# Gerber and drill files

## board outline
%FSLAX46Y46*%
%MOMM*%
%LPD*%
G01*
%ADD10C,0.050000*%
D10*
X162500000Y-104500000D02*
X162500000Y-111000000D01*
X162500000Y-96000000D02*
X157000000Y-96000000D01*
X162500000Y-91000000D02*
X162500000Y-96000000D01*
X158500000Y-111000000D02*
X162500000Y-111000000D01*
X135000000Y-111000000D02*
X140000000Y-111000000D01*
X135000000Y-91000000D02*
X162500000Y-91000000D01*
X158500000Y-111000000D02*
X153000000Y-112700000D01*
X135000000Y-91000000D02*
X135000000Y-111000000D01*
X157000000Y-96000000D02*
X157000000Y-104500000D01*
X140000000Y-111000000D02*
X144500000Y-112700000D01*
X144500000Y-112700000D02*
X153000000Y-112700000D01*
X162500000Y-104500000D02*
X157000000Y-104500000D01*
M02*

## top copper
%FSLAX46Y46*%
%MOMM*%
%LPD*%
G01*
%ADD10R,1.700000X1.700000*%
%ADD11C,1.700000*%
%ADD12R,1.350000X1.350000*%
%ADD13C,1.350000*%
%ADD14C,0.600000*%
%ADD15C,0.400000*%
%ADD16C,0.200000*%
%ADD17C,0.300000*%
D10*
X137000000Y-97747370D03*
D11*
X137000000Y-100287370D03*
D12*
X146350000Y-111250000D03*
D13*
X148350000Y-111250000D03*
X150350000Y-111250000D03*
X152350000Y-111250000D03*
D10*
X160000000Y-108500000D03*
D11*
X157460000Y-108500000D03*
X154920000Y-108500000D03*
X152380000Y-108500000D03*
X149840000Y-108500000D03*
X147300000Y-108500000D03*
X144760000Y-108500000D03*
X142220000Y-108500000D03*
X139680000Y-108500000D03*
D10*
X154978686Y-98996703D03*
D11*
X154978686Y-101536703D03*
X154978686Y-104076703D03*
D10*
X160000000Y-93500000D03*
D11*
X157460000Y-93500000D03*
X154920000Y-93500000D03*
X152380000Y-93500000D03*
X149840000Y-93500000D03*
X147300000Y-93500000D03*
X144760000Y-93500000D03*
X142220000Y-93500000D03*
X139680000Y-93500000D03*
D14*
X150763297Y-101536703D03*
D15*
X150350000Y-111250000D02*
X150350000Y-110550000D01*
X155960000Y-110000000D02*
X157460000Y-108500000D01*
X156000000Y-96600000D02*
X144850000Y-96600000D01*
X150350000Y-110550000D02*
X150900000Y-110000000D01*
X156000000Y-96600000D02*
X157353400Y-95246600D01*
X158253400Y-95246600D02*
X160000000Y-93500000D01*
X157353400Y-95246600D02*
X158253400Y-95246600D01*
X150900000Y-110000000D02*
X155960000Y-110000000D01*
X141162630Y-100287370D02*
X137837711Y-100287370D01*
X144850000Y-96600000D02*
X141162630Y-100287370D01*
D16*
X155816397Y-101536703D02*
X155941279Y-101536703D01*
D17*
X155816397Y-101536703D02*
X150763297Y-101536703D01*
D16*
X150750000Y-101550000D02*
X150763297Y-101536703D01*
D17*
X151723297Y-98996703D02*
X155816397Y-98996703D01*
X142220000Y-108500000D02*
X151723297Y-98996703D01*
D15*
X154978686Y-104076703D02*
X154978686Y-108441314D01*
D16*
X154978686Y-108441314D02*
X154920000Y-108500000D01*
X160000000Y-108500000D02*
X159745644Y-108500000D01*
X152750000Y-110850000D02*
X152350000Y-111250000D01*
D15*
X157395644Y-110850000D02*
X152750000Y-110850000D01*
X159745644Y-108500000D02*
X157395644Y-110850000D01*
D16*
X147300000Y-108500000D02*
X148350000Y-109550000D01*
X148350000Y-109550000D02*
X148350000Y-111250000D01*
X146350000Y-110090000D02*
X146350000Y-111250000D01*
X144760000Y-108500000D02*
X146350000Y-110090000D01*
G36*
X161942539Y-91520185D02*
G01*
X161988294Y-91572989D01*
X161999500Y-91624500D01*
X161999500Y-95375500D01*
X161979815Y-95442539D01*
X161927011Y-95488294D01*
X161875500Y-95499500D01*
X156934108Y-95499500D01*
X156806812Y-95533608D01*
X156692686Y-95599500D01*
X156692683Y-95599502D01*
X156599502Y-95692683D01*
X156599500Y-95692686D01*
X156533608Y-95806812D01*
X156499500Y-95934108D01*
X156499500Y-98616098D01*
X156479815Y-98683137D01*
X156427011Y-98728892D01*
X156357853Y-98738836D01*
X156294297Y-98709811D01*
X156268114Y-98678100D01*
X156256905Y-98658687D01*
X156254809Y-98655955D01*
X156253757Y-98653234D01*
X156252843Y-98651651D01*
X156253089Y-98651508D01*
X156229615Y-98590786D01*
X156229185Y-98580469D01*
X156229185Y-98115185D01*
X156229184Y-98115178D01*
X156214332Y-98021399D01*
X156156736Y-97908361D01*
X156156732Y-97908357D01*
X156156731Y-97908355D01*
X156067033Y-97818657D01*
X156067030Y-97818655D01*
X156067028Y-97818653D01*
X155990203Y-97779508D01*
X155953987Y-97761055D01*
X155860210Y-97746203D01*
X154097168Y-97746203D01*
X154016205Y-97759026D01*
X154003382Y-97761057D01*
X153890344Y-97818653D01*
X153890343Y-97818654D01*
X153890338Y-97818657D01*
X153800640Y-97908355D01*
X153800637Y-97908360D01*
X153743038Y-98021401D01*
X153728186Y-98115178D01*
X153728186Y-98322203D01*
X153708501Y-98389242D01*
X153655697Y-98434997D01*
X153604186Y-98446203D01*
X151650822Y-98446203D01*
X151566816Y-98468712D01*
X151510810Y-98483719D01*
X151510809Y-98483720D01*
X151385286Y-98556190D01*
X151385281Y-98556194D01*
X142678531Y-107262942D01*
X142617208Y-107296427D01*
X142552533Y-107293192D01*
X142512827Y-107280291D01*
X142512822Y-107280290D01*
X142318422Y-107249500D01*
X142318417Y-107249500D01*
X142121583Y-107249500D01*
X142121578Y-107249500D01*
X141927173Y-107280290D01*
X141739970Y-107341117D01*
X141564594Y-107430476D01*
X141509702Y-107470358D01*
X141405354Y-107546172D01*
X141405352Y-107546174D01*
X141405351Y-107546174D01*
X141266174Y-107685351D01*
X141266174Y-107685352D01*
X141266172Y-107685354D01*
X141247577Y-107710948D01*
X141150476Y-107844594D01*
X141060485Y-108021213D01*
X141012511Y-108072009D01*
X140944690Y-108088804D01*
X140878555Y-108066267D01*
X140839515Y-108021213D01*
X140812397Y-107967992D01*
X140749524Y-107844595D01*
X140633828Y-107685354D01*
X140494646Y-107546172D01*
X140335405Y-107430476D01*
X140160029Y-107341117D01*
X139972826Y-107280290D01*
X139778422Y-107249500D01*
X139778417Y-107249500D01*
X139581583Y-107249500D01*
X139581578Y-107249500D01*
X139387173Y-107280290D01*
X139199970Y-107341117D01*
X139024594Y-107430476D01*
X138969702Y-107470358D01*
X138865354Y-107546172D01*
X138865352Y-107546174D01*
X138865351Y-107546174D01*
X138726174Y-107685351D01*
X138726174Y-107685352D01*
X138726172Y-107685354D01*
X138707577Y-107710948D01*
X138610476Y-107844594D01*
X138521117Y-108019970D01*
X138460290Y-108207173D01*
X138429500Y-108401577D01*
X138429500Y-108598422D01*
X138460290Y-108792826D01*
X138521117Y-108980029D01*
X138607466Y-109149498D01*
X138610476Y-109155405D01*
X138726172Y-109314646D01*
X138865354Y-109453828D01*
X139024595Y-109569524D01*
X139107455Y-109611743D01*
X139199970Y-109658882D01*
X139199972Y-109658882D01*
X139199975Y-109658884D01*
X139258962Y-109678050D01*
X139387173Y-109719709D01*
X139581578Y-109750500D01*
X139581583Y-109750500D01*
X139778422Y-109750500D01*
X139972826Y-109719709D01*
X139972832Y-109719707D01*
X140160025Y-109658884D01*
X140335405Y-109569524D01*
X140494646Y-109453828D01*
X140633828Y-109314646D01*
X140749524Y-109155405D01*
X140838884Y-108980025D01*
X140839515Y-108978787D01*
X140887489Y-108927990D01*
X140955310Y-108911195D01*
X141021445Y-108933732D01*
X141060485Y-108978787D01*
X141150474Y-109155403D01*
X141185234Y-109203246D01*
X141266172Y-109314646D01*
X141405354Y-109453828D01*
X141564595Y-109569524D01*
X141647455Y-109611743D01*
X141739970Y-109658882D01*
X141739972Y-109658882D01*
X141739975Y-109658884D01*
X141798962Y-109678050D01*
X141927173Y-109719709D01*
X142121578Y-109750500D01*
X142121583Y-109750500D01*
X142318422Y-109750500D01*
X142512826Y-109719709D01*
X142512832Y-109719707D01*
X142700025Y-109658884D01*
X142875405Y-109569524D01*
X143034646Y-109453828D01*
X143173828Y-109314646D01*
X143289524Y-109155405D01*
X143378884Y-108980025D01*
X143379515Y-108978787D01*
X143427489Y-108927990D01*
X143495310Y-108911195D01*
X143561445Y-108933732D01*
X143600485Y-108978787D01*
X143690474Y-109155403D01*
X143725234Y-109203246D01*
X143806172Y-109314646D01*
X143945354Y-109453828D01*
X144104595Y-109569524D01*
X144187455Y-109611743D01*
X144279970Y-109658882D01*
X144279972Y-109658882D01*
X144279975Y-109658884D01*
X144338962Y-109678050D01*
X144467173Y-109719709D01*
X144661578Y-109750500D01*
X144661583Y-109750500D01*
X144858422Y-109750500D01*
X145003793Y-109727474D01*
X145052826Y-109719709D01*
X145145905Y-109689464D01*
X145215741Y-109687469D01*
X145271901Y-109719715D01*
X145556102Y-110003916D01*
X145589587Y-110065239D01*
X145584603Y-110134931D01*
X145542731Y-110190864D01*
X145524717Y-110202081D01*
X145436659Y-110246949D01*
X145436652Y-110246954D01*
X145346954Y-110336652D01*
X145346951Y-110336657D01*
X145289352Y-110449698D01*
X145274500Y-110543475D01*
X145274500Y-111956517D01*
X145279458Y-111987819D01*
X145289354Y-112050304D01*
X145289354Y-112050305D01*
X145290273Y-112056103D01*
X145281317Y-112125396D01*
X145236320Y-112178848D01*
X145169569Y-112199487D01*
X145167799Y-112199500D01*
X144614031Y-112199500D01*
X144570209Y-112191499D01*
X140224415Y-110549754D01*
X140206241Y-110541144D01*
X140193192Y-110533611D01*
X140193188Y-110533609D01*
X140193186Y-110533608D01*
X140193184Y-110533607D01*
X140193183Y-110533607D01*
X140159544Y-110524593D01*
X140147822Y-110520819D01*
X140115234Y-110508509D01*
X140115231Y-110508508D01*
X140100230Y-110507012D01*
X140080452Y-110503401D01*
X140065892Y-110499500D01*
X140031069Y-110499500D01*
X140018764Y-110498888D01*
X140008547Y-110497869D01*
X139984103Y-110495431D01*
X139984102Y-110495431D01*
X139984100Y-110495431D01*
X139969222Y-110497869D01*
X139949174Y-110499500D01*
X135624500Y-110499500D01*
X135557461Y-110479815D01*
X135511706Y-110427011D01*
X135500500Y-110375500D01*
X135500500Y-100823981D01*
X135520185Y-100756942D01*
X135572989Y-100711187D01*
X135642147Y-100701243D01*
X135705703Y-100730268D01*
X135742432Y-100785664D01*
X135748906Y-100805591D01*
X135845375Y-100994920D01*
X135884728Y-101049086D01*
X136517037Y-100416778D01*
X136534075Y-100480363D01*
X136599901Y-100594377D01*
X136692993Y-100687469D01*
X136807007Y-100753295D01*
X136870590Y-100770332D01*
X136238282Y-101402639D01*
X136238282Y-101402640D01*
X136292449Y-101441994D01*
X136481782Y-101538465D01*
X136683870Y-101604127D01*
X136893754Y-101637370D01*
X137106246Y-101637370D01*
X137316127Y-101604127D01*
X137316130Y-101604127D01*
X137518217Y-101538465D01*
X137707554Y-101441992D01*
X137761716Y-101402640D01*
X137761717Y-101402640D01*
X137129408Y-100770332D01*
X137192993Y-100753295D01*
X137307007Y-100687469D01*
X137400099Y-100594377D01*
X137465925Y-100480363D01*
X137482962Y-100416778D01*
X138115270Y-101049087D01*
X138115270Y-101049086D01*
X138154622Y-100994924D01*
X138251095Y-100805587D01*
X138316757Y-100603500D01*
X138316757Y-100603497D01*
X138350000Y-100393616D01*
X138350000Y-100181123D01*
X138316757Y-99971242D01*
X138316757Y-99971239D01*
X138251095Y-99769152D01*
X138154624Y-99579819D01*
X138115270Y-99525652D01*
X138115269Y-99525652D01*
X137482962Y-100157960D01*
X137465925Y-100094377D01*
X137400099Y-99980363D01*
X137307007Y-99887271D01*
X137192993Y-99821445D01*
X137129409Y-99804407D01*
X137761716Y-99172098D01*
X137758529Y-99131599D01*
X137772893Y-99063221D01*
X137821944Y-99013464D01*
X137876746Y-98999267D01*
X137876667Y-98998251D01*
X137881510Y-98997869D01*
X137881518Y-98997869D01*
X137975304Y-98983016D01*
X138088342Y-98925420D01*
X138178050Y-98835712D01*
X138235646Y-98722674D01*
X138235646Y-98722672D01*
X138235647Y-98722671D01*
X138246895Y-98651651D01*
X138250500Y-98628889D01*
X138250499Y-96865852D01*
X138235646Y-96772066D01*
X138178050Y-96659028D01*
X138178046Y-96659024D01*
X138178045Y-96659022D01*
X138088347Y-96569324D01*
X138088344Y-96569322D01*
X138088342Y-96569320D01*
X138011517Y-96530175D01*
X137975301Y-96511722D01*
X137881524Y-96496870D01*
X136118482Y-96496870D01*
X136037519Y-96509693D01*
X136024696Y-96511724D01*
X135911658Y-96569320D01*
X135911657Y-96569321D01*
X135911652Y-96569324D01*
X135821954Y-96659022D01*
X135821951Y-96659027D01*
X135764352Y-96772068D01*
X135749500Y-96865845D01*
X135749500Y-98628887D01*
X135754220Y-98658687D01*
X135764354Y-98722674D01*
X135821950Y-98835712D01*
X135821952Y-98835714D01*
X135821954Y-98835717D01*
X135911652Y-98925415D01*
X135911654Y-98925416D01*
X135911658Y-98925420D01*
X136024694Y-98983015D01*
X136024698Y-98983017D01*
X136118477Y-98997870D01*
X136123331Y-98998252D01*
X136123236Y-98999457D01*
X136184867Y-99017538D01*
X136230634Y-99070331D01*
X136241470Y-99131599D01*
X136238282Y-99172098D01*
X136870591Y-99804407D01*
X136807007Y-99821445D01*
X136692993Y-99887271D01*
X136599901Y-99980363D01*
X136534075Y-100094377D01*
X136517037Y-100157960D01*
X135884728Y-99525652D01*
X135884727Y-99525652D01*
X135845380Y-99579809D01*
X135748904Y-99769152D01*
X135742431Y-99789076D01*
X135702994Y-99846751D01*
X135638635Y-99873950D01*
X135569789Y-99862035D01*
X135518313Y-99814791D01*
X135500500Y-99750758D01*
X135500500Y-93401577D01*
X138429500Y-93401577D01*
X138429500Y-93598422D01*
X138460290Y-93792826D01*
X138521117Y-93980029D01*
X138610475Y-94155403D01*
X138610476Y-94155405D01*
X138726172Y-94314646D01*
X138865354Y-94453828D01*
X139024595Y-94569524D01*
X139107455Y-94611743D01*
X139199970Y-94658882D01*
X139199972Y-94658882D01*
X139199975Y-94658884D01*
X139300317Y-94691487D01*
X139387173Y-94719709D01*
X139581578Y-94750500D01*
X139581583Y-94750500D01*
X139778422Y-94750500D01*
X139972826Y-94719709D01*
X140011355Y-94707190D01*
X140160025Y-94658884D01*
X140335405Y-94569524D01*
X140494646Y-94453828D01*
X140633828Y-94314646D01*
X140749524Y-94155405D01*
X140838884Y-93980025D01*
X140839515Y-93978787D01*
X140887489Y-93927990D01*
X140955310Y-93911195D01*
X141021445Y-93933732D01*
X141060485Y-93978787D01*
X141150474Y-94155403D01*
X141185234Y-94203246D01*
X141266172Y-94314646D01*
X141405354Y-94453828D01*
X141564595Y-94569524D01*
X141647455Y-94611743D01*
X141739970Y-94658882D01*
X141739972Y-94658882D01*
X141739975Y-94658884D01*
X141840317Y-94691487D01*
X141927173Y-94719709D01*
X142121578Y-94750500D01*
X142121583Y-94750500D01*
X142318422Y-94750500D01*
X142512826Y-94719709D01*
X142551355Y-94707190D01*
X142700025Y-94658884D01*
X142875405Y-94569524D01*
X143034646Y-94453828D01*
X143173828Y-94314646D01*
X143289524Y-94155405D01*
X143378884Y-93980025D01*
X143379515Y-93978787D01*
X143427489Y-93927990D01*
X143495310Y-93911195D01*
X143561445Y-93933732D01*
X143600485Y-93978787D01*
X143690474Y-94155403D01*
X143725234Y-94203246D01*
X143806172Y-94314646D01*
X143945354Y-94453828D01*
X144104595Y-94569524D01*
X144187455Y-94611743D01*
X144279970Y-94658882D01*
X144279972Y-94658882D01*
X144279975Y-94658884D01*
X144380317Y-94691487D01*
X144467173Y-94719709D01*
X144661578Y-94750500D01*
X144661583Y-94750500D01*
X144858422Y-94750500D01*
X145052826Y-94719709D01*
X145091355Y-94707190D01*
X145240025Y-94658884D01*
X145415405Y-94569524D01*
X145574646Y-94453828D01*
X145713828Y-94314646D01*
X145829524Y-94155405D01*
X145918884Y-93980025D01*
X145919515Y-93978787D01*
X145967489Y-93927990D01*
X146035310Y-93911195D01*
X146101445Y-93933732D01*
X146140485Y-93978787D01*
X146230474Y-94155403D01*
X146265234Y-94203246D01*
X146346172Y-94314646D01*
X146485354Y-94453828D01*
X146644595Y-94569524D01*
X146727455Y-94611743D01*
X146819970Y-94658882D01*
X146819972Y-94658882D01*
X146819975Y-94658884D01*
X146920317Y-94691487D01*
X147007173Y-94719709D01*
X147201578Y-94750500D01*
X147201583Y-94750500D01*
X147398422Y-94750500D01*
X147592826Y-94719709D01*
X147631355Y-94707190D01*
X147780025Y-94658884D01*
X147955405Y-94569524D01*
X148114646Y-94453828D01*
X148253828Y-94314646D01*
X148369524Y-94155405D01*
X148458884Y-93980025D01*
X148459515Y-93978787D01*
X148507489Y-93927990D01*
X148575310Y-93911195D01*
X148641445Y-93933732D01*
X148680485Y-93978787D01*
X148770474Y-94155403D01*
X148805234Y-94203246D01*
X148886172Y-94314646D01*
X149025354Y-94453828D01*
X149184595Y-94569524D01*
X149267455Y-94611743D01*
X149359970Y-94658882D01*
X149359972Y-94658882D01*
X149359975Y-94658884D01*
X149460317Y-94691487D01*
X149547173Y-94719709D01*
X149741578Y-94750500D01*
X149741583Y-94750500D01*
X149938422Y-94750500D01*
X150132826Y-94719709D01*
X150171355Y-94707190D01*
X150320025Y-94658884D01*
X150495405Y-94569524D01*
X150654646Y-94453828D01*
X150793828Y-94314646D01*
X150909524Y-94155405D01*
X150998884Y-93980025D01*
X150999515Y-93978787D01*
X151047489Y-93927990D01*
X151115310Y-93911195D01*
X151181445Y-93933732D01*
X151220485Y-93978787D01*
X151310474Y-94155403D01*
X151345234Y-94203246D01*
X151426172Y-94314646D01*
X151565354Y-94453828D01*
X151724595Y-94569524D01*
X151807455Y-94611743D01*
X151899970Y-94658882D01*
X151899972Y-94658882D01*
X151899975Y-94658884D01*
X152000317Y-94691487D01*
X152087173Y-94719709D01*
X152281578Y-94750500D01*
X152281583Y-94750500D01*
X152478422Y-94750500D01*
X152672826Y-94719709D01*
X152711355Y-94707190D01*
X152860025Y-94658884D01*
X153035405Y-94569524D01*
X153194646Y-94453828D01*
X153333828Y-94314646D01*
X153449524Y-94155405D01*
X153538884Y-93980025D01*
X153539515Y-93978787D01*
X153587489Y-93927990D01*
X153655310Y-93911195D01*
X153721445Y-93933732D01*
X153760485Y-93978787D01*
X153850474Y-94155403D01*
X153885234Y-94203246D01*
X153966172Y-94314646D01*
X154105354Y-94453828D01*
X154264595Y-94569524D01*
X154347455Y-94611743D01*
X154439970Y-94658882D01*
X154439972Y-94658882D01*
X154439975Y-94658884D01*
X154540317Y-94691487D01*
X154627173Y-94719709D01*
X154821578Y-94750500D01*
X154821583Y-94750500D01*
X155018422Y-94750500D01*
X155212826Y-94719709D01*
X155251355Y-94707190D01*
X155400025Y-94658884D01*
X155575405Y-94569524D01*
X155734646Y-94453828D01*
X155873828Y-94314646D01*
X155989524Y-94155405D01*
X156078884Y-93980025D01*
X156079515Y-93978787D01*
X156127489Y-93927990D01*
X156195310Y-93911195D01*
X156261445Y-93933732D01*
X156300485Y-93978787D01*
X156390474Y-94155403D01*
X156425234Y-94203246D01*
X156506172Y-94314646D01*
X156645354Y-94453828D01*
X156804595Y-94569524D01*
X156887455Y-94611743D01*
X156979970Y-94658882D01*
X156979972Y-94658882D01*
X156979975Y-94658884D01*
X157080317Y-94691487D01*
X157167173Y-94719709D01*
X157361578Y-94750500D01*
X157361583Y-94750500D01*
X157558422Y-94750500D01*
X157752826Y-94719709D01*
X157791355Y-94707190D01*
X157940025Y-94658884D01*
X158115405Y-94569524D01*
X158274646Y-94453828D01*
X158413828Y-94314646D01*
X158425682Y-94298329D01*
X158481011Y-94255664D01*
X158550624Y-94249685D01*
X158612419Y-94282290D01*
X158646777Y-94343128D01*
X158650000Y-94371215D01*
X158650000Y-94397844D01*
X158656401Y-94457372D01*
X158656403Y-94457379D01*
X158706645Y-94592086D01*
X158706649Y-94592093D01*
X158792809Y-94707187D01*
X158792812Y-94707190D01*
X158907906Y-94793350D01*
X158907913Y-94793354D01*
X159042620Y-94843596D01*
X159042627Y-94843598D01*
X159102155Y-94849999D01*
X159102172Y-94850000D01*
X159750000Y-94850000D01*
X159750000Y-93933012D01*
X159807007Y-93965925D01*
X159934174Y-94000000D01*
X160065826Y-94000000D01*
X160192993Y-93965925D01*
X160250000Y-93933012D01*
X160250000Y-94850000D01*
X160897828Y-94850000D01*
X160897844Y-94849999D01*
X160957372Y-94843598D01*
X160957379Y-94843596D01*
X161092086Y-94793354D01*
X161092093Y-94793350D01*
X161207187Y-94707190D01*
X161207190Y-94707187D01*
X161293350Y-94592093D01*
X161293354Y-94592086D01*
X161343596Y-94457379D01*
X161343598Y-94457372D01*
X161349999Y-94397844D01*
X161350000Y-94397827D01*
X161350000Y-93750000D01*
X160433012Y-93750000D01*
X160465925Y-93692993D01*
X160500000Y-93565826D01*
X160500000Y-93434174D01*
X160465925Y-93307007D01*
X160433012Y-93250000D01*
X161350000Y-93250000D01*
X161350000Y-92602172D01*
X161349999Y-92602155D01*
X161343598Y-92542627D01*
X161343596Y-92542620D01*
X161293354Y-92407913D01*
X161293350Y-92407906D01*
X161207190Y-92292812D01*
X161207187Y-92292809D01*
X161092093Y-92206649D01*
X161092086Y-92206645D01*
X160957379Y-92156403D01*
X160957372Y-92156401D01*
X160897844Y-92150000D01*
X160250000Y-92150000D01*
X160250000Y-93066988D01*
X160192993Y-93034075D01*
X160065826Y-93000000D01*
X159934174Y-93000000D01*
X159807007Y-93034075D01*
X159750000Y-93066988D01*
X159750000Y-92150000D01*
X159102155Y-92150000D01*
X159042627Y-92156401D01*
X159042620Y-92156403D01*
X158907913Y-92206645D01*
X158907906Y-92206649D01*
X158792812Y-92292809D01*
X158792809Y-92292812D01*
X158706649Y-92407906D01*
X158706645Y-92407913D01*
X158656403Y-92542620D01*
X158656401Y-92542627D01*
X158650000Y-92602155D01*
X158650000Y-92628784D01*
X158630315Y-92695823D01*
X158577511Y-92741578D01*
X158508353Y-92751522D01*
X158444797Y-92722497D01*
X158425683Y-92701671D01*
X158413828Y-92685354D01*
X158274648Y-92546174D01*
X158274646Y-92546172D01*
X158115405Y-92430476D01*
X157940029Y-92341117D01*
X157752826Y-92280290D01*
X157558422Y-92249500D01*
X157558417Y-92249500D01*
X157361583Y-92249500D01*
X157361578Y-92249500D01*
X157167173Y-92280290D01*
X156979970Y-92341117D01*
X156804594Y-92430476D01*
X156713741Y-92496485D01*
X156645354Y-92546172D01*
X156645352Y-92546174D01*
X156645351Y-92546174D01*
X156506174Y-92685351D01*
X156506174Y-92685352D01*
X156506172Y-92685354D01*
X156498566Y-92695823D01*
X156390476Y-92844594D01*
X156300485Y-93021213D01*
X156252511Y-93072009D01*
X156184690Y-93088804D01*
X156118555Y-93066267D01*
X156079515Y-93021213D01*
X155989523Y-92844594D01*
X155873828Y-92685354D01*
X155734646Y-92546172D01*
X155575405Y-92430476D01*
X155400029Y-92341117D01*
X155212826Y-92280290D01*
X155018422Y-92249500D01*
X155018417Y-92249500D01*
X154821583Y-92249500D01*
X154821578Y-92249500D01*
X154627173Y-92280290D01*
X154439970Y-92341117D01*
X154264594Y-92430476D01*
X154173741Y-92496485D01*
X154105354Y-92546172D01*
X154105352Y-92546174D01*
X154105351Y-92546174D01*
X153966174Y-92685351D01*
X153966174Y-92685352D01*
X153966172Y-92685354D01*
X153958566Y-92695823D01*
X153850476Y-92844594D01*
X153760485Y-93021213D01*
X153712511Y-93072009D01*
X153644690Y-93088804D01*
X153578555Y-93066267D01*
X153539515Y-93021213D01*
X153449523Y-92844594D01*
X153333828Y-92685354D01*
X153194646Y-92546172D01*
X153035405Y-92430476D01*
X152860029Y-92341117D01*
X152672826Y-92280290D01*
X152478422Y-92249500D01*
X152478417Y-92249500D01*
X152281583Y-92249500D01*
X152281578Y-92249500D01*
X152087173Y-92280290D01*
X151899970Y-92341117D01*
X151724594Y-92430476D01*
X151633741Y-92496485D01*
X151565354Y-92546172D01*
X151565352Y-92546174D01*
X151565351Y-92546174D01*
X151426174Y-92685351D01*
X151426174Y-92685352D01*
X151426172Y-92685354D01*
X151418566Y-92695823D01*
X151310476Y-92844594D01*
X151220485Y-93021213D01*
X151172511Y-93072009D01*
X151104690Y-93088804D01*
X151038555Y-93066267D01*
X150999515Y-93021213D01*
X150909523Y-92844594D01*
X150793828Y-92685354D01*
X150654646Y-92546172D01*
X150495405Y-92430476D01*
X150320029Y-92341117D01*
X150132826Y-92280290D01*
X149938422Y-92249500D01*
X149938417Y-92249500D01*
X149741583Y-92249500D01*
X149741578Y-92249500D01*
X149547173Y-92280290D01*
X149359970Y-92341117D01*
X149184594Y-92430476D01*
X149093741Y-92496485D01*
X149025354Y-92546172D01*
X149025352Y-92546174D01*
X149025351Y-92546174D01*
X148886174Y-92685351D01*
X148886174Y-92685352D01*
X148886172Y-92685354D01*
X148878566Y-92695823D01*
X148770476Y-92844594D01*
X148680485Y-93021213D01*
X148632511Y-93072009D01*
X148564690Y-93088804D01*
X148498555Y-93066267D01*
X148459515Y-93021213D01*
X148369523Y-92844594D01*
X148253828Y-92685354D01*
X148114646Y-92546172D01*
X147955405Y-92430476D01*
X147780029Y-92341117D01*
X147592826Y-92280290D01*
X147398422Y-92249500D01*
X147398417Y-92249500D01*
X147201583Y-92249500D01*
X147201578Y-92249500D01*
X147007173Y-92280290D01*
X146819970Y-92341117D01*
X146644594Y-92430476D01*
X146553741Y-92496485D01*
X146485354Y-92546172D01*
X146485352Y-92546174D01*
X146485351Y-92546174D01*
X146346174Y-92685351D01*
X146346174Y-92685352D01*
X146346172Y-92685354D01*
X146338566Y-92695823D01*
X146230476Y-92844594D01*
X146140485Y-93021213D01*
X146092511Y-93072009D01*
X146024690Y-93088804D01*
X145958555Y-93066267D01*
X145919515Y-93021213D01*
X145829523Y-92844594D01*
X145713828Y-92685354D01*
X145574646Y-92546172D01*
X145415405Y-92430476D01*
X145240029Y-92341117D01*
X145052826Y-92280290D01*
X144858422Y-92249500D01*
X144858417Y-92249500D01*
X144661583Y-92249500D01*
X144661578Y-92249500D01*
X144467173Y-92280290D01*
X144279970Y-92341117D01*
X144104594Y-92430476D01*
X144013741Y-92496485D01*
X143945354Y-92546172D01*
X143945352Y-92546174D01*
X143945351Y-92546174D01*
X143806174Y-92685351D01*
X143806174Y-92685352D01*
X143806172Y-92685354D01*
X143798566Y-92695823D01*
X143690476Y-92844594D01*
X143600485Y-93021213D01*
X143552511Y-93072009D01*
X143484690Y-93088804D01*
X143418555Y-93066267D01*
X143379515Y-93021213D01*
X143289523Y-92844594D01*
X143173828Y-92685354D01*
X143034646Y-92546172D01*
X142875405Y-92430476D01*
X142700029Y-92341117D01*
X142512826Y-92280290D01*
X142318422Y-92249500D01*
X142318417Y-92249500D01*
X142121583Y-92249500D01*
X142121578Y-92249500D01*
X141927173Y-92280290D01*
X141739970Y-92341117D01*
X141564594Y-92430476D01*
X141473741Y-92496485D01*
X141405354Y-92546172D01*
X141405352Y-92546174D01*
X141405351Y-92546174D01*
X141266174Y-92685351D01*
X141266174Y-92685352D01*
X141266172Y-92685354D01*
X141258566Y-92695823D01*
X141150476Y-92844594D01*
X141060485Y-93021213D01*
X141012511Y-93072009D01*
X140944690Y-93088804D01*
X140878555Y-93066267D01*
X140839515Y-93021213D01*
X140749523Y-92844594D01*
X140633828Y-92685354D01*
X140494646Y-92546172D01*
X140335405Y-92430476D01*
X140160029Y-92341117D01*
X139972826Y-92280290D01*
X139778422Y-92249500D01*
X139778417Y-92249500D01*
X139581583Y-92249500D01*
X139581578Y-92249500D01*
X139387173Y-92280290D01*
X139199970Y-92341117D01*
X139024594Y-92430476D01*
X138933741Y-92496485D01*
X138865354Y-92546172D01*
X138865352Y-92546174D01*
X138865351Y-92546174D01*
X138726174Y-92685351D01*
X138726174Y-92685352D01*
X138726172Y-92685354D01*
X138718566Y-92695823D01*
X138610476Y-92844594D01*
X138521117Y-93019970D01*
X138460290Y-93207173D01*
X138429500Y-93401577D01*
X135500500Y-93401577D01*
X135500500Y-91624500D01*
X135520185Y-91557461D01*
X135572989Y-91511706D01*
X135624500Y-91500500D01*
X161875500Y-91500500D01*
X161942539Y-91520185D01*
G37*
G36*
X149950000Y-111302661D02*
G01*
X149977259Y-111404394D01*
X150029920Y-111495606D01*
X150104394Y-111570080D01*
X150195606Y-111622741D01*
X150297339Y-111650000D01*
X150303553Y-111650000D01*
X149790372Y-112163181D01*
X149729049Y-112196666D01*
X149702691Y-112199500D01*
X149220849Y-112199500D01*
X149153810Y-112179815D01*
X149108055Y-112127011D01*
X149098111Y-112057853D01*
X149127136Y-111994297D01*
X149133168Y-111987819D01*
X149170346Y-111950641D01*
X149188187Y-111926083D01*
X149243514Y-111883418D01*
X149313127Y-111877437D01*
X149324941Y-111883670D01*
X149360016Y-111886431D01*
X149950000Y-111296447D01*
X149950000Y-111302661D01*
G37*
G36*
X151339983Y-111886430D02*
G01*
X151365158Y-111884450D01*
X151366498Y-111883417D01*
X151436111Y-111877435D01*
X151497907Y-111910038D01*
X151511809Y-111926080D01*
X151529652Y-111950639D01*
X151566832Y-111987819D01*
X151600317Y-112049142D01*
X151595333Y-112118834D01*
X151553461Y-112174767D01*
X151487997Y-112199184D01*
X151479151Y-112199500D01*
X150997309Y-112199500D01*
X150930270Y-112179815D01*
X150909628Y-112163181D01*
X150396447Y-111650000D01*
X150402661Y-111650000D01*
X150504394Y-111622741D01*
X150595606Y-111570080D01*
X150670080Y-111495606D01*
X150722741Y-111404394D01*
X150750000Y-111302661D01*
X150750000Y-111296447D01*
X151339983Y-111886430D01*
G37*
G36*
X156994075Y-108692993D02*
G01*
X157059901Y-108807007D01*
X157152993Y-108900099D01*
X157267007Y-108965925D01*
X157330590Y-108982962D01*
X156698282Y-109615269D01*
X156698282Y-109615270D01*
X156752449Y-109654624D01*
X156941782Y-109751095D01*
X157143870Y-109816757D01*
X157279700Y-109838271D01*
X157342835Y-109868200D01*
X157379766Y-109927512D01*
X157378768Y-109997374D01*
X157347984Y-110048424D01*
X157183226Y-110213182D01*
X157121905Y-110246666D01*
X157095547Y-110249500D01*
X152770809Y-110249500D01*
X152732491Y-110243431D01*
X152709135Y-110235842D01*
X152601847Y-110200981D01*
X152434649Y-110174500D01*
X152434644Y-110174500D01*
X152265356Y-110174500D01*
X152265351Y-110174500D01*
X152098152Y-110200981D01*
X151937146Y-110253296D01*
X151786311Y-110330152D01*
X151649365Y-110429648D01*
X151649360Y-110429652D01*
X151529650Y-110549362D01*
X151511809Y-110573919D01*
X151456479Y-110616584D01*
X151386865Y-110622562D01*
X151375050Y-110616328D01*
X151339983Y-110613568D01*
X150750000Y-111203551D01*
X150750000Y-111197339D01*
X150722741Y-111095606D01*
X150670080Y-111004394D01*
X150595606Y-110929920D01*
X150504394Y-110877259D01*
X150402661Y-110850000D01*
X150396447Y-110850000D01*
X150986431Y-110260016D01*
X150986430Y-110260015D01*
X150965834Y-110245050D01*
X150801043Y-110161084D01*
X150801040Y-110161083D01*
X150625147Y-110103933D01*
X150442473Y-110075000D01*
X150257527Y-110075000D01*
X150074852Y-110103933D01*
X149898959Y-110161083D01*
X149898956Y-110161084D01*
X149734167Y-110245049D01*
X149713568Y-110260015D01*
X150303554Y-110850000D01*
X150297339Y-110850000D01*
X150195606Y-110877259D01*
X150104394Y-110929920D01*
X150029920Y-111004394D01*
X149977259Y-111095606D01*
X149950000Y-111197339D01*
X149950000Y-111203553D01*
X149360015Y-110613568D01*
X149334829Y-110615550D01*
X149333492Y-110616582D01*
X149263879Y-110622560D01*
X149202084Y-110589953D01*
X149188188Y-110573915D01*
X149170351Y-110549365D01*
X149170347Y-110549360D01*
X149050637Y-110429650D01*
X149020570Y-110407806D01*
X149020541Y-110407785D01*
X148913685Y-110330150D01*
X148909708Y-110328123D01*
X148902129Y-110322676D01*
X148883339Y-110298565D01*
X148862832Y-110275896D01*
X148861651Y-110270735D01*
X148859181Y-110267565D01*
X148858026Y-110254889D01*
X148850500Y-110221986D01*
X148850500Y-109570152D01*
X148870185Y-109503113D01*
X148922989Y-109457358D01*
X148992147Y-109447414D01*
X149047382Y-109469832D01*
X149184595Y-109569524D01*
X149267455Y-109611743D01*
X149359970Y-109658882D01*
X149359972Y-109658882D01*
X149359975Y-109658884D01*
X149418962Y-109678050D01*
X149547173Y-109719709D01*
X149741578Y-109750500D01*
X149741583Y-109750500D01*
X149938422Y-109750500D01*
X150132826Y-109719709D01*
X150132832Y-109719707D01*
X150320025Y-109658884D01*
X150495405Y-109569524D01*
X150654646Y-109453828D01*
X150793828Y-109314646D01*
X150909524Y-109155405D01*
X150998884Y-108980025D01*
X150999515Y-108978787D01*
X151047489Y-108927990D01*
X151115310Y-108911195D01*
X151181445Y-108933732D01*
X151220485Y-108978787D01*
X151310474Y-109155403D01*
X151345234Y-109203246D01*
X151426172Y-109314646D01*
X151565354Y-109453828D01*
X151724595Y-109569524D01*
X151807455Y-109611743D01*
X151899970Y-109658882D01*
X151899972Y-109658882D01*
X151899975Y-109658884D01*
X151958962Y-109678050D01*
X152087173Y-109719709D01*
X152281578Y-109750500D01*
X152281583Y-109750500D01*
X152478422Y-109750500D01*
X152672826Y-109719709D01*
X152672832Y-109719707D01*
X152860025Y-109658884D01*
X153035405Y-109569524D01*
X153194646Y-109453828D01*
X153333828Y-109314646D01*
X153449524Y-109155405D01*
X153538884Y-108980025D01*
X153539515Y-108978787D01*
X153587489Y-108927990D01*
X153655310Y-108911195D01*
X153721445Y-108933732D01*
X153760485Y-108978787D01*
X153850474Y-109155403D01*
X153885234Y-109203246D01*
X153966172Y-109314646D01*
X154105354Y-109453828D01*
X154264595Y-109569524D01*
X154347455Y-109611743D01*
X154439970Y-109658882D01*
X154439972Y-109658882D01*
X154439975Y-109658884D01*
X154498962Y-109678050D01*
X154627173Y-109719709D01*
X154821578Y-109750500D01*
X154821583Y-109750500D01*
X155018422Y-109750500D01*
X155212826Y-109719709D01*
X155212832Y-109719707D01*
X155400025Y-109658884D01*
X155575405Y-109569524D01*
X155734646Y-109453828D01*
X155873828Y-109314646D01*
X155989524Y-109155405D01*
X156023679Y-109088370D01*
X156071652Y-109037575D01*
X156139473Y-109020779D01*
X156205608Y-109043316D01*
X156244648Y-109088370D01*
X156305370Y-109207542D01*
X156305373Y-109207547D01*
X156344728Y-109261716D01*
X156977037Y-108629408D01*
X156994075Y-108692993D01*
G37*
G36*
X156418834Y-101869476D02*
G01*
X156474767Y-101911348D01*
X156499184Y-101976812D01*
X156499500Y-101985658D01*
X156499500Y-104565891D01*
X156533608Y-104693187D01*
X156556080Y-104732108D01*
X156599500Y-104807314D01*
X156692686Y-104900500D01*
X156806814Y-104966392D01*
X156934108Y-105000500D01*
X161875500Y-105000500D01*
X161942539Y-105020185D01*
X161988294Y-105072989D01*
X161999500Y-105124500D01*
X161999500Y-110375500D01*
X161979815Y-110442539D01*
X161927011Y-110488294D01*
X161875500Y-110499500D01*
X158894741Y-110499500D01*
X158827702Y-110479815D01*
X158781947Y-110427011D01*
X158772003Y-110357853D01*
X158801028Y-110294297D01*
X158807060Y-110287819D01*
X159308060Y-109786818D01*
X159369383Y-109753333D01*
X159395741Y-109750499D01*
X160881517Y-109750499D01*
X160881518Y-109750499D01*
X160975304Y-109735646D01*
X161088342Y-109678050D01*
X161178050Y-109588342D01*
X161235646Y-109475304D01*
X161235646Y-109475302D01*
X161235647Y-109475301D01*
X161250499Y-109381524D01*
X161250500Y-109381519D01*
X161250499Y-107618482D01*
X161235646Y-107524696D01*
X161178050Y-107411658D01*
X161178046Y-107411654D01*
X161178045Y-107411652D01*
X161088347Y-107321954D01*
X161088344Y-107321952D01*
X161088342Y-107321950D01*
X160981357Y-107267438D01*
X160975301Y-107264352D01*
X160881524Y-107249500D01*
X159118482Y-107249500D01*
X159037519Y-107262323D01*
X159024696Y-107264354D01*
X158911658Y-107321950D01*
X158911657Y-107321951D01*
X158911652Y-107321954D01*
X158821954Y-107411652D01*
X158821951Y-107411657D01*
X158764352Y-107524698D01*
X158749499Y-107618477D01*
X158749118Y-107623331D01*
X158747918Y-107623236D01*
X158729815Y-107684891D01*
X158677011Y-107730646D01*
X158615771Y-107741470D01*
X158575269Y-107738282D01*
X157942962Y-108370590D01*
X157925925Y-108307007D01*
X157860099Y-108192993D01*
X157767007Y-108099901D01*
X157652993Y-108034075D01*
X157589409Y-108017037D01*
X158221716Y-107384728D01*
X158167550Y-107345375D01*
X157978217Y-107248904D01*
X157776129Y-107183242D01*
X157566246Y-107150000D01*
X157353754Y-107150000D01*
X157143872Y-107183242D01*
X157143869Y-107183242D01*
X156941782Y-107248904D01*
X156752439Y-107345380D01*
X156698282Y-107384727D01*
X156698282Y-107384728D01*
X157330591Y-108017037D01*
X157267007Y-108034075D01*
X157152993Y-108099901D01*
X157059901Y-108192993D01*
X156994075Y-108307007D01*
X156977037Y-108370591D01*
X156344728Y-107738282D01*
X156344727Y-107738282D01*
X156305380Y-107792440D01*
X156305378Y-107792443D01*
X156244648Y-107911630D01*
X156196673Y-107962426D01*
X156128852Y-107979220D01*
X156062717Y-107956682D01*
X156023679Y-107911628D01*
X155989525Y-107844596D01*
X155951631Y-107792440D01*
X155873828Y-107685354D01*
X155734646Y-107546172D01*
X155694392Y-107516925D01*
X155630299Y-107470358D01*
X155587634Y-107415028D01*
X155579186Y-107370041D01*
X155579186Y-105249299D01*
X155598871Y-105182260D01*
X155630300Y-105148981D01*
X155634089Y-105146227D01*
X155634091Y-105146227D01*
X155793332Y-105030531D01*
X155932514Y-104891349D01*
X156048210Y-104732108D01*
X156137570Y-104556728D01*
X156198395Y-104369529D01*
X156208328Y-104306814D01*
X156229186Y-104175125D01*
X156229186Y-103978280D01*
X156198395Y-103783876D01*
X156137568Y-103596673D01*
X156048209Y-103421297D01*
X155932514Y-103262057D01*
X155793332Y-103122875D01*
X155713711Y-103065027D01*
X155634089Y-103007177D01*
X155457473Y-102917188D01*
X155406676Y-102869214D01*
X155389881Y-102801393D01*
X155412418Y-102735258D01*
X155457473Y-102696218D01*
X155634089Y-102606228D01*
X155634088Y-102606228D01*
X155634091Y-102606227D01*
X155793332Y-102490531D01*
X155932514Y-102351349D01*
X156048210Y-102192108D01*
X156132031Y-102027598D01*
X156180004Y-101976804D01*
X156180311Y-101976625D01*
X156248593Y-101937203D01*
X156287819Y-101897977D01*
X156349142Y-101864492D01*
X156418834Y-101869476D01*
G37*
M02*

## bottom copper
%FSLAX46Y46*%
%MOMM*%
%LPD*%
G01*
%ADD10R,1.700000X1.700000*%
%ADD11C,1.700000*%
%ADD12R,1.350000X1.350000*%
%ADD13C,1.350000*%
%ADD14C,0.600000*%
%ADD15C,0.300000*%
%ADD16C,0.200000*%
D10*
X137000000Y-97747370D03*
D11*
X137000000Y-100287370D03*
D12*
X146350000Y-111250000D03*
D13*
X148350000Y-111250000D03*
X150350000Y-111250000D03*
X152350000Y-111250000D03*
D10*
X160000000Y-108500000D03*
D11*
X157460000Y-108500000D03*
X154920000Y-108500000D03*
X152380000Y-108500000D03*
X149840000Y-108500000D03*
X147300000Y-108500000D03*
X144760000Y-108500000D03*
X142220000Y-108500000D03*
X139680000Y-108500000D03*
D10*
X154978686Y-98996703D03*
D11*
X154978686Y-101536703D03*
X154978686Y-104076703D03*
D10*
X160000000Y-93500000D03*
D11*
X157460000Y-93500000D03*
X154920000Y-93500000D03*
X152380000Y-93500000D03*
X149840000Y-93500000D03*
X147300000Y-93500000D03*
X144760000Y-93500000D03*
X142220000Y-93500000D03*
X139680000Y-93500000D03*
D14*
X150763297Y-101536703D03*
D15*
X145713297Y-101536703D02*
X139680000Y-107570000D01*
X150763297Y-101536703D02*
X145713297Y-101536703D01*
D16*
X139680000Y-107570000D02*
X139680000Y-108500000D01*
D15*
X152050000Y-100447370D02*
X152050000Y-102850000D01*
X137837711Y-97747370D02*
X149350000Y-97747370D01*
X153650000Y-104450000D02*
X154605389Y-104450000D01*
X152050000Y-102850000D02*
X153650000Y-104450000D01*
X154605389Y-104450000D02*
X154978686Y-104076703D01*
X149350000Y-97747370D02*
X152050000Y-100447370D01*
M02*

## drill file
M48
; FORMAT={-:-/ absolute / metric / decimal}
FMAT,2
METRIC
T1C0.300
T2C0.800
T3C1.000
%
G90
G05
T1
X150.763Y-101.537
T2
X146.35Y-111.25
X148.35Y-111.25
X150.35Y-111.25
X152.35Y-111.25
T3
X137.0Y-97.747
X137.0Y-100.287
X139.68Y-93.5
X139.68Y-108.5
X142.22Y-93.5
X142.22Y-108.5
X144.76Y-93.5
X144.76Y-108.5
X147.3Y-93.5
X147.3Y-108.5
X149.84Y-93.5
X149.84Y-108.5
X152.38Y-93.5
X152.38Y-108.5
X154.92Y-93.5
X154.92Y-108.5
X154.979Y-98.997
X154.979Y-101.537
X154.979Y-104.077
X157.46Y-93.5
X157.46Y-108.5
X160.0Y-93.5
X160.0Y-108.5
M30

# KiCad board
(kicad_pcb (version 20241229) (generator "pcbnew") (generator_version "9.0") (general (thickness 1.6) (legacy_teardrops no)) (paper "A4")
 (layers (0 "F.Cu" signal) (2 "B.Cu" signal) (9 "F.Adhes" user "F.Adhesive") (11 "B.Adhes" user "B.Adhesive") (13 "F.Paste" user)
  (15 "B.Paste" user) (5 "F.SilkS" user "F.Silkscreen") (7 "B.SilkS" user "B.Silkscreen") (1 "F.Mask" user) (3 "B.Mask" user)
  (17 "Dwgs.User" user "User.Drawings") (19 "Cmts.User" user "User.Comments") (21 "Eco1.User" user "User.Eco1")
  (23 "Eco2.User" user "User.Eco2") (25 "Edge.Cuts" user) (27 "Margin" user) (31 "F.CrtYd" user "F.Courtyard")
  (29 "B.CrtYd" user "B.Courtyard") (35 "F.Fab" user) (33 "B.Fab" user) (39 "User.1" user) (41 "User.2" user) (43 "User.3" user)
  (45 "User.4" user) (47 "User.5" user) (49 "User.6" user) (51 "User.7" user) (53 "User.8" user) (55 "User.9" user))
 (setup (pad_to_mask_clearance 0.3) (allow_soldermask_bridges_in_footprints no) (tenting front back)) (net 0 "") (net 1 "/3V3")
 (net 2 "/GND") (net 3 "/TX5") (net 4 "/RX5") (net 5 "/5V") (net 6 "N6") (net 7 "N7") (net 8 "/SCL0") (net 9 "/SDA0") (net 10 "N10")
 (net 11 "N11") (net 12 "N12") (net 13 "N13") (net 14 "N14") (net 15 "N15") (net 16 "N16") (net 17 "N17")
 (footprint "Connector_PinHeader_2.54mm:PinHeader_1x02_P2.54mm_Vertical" (layer "F.Cu") (at 140 97.74737)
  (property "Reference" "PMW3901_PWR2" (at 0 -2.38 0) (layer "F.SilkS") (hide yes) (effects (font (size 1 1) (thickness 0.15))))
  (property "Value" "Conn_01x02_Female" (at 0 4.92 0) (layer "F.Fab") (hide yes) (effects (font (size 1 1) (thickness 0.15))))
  (pad "1" thru_hole rect (at -3 0) (size 1.7 1.7) (drill 1) (layers "*.Cu" "*.Mask") (remove_unused_layers no) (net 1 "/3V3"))
  (pad "2" thru_hole circle (at -3 2.54) (size 1.7 1.7) (drill 1) (layers "*.Cu" "*.Mask") (remove_unused_layers no) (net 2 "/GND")))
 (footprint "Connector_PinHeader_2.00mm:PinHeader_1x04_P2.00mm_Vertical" (layer "F.Cu") (at 146.35 111.25 90)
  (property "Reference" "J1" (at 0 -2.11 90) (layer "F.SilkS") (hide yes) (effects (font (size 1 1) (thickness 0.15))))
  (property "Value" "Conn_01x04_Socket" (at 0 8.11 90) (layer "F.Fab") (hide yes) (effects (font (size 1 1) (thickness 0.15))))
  (pad "1" thru_hole rect (at 0 0 90) (size 1.35 1.35) (drill 0.8) (layers "*.Cu" "*.Mask") (remove_unused_layers no) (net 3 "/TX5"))
  (pad "2" thru_hole circle (at 0 2 90) (size 1.35 1.35) (drill 0.8) (layers "*.Cu" "*.Mask") (remove_unused_layers no) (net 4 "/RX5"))
  (pad "3" thru_hole circle (at 0 4 90) (size 1.35 1.35) (drill 0.8) (layers "*.Cu" "*.Mask") (remove_unused_layers no) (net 2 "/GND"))
  (pad "4" thru_hole circle (at 0 6 90) (size 1.35 1.35) (drill 0.8) (layers "*.Cu" "*.Mask") (remove_unused_layers no) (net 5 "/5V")))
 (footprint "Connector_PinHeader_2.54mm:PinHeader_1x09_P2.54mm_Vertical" (layer "F.Cu") (at 160 108.5 -90)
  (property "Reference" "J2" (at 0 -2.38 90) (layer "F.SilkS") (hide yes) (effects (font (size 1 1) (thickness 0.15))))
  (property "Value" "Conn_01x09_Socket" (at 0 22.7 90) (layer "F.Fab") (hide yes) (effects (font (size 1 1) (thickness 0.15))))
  (pad "1" thru_hole rect (at 0 0 270) (size 1.7 1.7) (drill 1) (layers "*.Cu" "*.Mask") (remove_unused_layers no) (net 5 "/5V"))
  (pad "2" thru_hole circle (at 0 2.54 270) (size 1.7 1.7) (drill 1) (layers "*.Cu" "*.Mask") (remove_unused_layers no) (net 2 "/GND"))
  (pad "3" thru_hole circle (at 0 5.08 270) (size 1.7 1.7) (drill 1) (layers "*.Cu" "*.Mask") (remove_unused_layers no) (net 1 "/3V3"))
  (pad "4" thru_hole circle (at 0 7.62 270) (size 1.7 1.7) (drill 1) (layers "*.Cu" "*.Mask") (remove_unused_layers no) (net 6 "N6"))
  (pad "5" thru_hole circle (at 0 10.16 270) (size 1.7 1.7) (drill 1) (layers "*.Cu" "*.Mask") (remove_unused_layers no) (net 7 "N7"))
  (pad "6" thru_hole circle (at 0 12.7 270) (size 1.7 1.7) (drill 1) (layers "*.Cu" "*.Mask") (remove_unused_layers no) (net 4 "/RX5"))
  (pad "7" thru_hole circle (at 0 15.24 270) (size 1.7 1.7) (drill 1) (layers "*.Cu" "*.Mask") (remove_unused_layers no) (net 3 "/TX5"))
  (pad "8" thru_hole circle (at 0 17.78 270) (size 1.7 1.7) (drill 1) (layers "*.Cu" "*.Mask") (remove_unused_layers no) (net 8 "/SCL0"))
  (pad "9" thru_hole circle (at 0 20.32 270) (size 1.7 1.7) (drill 1) (layers "*.Cu" "*.Mask") (remove_unused_layers no) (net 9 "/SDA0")))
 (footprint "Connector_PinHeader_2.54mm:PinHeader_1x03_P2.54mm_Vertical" (layer "F.Cu") (at 154.251467 98.996703)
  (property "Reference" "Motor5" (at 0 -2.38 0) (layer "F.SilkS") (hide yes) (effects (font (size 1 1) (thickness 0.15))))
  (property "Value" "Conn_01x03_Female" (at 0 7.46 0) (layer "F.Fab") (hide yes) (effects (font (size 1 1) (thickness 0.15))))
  (pad "1" thru_hole rect (at 0.727219 0) (size 1.7 1.7) (drill 1) (layers "*.Cu" "*.Mask") (remove_unused_layers no) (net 8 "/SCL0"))
  (pad "2" thru_hole circle (at 0.727219 2.54) (size 1.7 1.7) (drill 1) (layers "*.Cu" "*.Mask") (remove_unused_layers no) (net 9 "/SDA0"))
  (pad "3" thru_hole circle (at 0.727219 5.08) (size 1.7 1.7) (drill 1) (layers "*.Cu" "*.Mask") (remove_unused_layers no) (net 1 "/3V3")))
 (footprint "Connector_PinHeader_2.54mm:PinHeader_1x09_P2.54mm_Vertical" (layer "F.Cu") (at 160 93.5 -90)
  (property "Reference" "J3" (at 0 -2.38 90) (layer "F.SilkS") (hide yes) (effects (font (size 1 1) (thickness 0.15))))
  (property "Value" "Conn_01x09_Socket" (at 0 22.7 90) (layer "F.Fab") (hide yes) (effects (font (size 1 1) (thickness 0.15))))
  (pad "1" thru_hole rect (at 0 0 270) (size 1.7 1.7) (drill 1) (layers "*.Cu" "*.Mask") (remove_unused_layers no) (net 2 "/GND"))
  (pad "2" thru_hole circle (at 0 2.54 270) (size 1.7 1.7) (drill 1) (layers "*.Cu" "*.Mask") (remove_unused_layers no) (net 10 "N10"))
  (pad "3" thru_hole circle (at 0 5.08 270) (size 1.7 1.7) (drill 1) (layers "*.Cu" "*.Mask") (remove_unused_layers no) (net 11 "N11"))
  (pad "4" thru_hole circle (at 0 7.62 270) (size 1.7 1.7) (drill 1) (layers "*.Cu" "*.Mask") (remove_unused_layers no) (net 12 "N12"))
  (pad "5" thru_hole circle (at 0 10.16 270) (size 1.7 1.7) (drill 1) (layers "*.Cu" "*.Mask") (remove_unused_layers no) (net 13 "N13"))
  (pad "6" thru_hole circle (at 0 12.7 270) (size 1.7 1.7) (drill 1) (layers "*.Cu" "*.Mask") (remove_unused_layers no) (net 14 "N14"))
  (pad "7" thru_hole circle (at 0 15.24 270) (size 1.7 1.7) (drill 1) (layers "*.Cu" "*.Mask") (remove_unused_layers no) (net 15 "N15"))
  (pad "8" thru_hole circle (at 0 17.78 270) (size 1.7 1.7) (drill 1) (layers "*.Cu" "*.Mask") (remove_unused_layers no) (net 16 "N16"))
  (pad "9" thru_hole circle (at 0 20.32 270) (size 1.7 1.7) (drill 1) (layers "*.Cu" "*.Mask") (remove_unused_layers no) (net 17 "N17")))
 (gr_line (start 162.5 104.5) (end 162.5 111) (stroke (width 0.05) (type solid)) (layer "Edge.Cuts"))
 (gr_line (start 162.5 96) (end 157 96) (stroke (width 0.05) (type solid)) (layer "Edge.Cuts"))
 (gr_line (start 162.5 91) (end 162.5 96) (stroke (width 0.05) (type solid)) (layer "Edge.Cuts"))
 (gr_line (start 158.5 111) (end 162.5 111) (stroke (width 0.05) (type solid)) (layer "Edge.Cuts"))
 (gr_line (start 135 111) (end 140 111) (stroke (width 0.05) (type solid)) (layer "Edge.Cuts"))
 (gr_line (start 135 91) (end 162.5 91) (stroke (width 0.05) (type solid)) (layer "Edge.Cuts"))
 (gr_line (start 158.5 111) (end 153 112.7) (stroke (width 0.05) (type solid)) (layer "Edge.Cuts"))
 (gr_line (start 135 91) (end 135 111) (stroke (width 0.05) (type solid)) (layer "Edge.Cuts"))
 (gr_line (start 157 96) (end 157 104.5) (stroke (width 0.05) (type solid)) (layer "Edge.Cuts"))
 (gr_line (start 140 111) (end 144.5 112.7) (stroke (width 0.05) (type default)) (layer "Edge.Cuts"))
 (gr_line (start 144.5 112.7) (end 153 112.7) (stroke (width 0.05) (type solid)) (layer "Edge.Cuts"))
 (gr_line (start 162.5 104.5) (end 157 104.5) (stroke (width 0.05) (type solid)) (layer "Edge.Cuts"))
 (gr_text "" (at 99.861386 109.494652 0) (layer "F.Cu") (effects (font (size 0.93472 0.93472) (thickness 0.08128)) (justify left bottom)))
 (segment (start 150.35 111.25) (end 150.35 110.55) (width 0.4) (layer "F.Cu") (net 2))
 (segment (start 155.96 110) (end 157.46 108.5) (width 0.4) (layer "F.Cu") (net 2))
 (segment (start 156 96.6) (end 144.85 96.6) (width 0.4) (layer "F.Cu") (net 2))
 (segment (start 150.35 110.55) (end 150.9 110) (width 0.4) (layer "F.Cu") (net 2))
 (segment (start 156 96.6) (end 157.3534 95.2466) (width 0.4) (layer "F.Cu") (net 2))
 (segment (start 158.2534 95.2466) (end 160 93.5) (width 0.4) (layer "F.Cu") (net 2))
 (segment (start 157.3534 95.2466) (end 158.2534 95.2466) (width 0.4) (layer "F.Cu") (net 2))
 (segment (start 150.9 110) (end 155.96 110) (width 0.4) (layer "F.Cu") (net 2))
 (segment (start 141.16263 100.28737) (end 137.837711 100.28737) (width 0.4) (layer "F.Cu") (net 2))
 (segment (start 144.85 96.6) (end 141.16263 100.28737) (width 0.4) (layer "F.Cu") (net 2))
 (segment (start 155.816397 101.536703) (end 155.941279 101.536703) (width 0.2) (layer "F.Cu") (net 9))
 (segment (start 155.816397 101.536703) (end 150.763297 101.536703) (width 0.3) (layer "F.Cu") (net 9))
 (segment (start 150.75 101.55) (end 150.763297 101.536703) (width 0.2) (layer "F.Cu") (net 9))
 (via (at 150.763297 101.536703) (size 0.6) (drill 0.3) (layers "F.Cu" "B.Cu") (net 9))
 (segment (start 145.713297 101.536703) (end 139.68 107.57) (width 0.3) (layer "B.Cu") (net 9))
 (segment (start 150.763297 101.536703) (end 145.713297 101.536703) (width 0.3) (layer "B.Cu") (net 9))
 (segment (start 139.68 107.57) (end 139.68 108.5) (width 0.2) (layer "B.Cu") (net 9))
 (segment (start 151.723297 98.996703) (end 155.816397 98.996703) (width 0.3) (layer "F.Cu") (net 8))
 (segment (start 142.22 108.5) (end 151.723297 98.996703) (width 0.3) (layer "F.Cu") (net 8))
 (segment (start 154.978686 104.076703) (end 154.978686 108.441314) (width 0.4) (layer "F.Cu") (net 1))
 (segment (start 154.978686 108.441314) (end 154.92 108.5) (width 0.2) (layer "F.Cu") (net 1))
 (segment (start 152.05 100.44737) (end 152.05 102.85) (width 0.3) (layer "B.Cu") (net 1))
 (segment (start 137.837711 97.74737) (end 149.35 97.74737) (width 0.3) (layer "B.Cu") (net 1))
 (segment (start 153.65 104.45) (end 154.605389 104.45) (width 0.3) (layer "B.Cu") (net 1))
 (segment (start 152.05 102.85) (end 153.65 104.45) (width 0.3) (layer "B.Cu") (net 1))
 (segment (start 154.605389 104.45) (end 154.978686 104.076703) (width 0.3) (layer "B.Cu") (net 1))
 (segment (start 149.35 97.74737) (end 152.05 100.44737) (width 0.3) (layer "B.Cu") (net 1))
 (segment (start 160 108.5) (end 159.745644 108.5) (width 0.2) (layer "F.Cu") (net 5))
 (segment (start 152.75 110.85) (end 152.35 111.25) (width 0.2) (layer "F.Cu") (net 5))
 (segment (start 157.395644 110.85) (end 152.75 110.85) (width 0.4) (layer "F.Cu") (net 5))
 (segment (start 159.745644 108.5) (end 157.395644 110.85) (width 0.4) (layer "F.Cu") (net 5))
 (segment (start 147.3 108.5) (end 148.35 109.55) (width 0.2) (layer "F.Cu") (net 4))
 (segment (start 148.35 109.55) (end 148.35 111.25) (width 0.2) (layer "F.Cu") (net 4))
 (segment (start 146.35 110.09) (end 146.35 111.25) (width 0.2) (layer "F.Cu") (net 3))
 (segment (start 144.76 108.5) (end 146.35 110.09) (width 0.2) (layer "F.Cu") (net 3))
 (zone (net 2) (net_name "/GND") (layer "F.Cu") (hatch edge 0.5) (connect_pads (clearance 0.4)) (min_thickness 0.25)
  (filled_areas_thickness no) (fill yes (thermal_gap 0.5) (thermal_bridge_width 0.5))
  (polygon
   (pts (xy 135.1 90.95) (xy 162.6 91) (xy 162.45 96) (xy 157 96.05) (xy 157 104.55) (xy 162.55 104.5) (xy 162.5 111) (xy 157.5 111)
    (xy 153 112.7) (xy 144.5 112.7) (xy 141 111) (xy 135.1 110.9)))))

